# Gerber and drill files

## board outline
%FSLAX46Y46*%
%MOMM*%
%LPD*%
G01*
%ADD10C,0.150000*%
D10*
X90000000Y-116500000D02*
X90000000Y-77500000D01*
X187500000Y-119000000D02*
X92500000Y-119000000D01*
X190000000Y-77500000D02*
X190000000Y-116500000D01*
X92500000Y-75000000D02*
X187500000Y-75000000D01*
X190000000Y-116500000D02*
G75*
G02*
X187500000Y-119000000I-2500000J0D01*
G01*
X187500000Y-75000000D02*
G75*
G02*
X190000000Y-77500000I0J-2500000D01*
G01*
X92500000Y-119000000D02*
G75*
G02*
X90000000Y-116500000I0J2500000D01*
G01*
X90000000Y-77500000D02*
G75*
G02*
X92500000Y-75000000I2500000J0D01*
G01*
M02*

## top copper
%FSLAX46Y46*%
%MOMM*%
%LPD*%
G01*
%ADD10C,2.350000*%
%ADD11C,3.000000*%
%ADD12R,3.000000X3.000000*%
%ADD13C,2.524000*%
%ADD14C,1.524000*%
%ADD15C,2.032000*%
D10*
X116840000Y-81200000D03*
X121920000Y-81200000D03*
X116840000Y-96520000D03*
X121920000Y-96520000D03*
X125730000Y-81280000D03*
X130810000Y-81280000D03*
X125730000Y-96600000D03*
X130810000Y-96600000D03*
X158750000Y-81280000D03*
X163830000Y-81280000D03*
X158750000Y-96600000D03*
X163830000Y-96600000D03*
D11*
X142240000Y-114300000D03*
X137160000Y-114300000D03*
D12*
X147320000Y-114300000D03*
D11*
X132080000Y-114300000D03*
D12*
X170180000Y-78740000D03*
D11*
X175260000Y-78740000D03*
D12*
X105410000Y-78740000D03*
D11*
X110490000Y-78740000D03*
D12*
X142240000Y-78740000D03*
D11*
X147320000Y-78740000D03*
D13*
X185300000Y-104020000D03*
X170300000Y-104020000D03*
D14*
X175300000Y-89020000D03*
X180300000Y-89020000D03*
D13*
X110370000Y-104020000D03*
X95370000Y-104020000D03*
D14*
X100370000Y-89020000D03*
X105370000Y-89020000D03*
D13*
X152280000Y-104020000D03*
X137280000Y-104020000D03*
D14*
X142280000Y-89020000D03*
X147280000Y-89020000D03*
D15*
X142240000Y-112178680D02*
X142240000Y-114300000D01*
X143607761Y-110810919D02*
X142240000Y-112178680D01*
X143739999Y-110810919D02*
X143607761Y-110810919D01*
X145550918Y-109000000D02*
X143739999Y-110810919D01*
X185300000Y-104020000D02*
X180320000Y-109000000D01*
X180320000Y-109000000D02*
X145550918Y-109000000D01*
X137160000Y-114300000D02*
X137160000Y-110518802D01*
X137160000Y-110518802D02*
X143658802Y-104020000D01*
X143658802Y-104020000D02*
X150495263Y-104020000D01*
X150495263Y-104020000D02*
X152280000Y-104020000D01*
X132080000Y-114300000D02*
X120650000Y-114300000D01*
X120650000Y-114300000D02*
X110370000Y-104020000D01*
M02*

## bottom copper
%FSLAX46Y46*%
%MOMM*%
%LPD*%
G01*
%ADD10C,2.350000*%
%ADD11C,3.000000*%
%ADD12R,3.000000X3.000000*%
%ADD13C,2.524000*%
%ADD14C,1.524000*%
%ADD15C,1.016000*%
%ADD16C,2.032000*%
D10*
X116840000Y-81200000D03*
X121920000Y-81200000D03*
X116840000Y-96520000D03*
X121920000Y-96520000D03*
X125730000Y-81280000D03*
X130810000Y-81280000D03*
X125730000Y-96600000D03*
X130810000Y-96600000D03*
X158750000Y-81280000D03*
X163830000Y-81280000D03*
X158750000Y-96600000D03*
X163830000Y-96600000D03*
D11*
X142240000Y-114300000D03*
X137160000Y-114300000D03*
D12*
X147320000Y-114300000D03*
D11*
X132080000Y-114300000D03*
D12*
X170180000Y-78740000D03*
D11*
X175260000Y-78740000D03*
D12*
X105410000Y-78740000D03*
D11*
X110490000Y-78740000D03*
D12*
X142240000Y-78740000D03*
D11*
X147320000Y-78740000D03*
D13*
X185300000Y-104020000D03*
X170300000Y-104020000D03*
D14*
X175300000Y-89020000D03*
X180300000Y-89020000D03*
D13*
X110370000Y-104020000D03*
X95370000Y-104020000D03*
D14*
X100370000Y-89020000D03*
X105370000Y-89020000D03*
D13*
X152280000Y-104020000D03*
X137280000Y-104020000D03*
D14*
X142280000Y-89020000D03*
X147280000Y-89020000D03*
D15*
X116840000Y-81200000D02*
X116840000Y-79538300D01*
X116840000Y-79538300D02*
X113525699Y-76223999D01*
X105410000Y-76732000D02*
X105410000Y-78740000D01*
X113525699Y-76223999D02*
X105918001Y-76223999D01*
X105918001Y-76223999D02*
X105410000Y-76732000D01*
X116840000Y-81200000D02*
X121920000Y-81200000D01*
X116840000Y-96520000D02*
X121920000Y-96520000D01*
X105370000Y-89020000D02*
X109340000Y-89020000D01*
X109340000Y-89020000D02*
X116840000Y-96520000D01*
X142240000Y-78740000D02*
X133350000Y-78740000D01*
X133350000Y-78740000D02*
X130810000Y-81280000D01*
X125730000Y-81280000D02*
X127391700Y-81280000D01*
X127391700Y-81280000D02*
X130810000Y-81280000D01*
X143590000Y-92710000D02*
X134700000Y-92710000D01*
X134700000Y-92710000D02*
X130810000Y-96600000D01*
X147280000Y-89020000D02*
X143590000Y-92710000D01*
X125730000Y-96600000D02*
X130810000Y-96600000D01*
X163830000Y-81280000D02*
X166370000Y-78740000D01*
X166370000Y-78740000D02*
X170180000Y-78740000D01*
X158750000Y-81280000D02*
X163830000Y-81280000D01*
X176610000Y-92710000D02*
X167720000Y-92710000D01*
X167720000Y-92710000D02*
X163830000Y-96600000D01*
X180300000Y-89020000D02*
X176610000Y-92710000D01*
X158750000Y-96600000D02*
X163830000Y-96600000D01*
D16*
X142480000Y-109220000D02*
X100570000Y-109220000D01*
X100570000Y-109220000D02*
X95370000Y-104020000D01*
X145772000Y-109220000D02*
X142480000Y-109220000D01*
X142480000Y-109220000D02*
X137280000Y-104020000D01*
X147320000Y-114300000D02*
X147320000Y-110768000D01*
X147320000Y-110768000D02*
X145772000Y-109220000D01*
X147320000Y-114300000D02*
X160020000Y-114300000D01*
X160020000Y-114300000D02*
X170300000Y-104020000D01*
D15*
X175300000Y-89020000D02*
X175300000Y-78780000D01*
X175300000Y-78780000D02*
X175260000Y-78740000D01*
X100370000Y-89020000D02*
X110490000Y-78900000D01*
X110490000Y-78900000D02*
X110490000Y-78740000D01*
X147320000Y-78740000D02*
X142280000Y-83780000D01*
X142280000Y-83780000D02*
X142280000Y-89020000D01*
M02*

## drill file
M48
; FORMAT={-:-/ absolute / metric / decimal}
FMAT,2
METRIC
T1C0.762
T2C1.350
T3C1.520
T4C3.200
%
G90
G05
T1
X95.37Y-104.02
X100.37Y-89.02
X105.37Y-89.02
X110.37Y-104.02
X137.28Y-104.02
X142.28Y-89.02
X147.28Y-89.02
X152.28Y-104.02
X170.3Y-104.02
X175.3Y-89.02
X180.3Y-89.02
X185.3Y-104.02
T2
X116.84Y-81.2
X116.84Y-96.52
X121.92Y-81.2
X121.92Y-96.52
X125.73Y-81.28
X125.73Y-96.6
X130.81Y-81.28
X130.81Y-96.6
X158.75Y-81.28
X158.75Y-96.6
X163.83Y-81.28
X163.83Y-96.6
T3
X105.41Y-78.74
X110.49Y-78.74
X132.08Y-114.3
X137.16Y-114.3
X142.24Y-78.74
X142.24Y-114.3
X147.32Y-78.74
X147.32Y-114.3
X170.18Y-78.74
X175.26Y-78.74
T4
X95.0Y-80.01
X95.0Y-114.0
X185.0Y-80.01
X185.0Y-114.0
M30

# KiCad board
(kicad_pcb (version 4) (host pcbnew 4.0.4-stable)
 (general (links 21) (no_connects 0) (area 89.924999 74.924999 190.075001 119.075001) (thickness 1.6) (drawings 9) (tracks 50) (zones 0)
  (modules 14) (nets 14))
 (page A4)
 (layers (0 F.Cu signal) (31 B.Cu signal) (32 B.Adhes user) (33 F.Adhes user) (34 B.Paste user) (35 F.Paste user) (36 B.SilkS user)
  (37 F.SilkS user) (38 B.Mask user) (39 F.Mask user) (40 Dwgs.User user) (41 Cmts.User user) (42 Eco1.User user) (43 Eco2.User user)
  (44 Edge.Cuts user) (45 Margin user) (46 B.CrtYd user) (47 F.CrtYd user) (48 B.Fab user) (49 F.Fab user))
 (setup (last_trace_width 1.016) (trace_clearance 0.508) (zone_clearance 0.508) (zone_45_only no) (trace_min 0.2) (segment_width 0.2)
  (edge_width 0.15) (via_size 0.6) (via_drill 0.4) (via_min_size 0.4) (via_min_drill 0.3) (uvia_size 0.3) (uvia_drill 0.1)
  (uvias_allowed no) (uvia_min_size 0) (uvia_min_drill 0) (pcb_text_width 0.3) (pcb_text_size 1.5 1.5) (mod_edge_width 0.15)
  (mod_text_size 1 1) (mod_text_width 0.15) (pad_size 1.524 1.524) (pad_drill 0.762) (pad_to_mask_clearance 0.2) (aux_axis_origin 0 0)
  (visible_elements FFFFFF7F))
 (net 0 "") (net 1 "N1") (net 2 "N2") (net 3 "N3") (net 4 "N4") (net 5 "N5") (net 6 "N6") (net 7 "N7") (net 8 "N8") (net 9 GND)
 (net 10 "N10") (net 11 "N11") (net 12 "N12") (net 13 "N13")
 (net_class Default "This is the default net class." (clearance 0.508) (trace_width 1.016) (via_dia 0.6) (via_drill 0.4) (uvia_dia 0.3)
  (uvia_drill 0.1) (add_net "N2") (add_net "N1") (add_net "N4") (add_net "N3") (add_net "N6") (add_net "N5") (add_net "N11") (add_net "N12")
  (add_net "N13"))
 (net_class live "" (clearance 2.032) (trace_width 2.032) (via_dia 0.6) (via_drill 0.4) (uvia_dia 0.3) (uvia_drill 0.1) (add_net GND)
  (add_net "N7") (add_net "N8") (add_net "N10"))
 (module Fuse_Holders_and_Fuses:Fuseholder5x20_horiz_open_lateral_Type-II (layer F.Cu) (at 116.84 96.52 90)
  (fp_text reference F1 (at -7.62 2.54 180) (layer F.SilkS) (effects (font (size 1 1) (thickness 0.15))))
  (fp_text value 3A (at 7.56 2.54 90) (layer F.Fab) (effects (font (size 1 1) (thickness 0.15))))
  (pad 2 thru_hole circle (at 15.32 0 90) (size 2.35 2.35) (drill 1.35) (layers *.Cu *.Mask) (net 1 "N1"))
  (pad 2 thru_hole circle (at 15.32 5.08 90) (size 2.35 2.35) (drill 1.35) (layers *.Cu *.Mask) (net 1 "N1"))
  (pad 1 thru_hole circle (at 0 0 90) (size 2.35 2.35) (drill 1.35) (layers *.Cu *.Mask) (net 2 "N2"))
  (pad 1 thru_hole circle (at 0 5.08 90) (size 2.35 2.35) (drill 1.35) (layers *.Cu *.Mask) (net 2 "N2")))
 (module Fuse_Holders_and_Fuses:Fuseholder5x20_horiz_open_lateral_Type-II (layer F.Cu) (at 125.73 96.6 90)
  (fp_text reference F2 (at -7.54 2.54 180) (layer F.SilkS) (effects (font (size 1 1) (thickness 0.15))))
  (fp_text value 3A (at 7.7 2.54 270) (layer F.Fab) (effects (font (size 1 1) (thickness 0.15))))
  (pad 2 thru_hole circle (at 15.32 0 90) (size 2.35 2.35) (drill 1.35) (layers *.Cu *.Mask) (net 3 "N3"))
  (pad 2 thru_hole circle (at 15.32 5.08 90) (size 2.35 2.35) (drill 1.35) (layers *.Cu *.Mask) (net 3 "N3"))
  (pad 1 thru_hole circle (at 0 0 90) (size 2.35 2.35) (drill 1.35) (layers *.Cu *.Mask) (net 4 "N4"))
  (pad 1 thru_hole circle (at 0 5.08 90) (size 2.35 2.35) (drill 1.35) (layers *.Cu *.Mask) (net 4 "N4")))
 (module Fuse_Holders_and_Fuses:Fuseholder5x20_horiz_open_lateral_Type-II (layer F.Cu) (at 158.75 96.6 90)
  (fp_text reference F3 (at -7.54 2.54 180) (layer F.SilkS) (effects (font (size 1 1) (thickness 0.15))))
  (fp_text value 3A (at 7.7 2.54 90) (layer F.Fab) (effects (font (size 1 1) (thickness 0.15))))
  (pad 2 thru_hole circle (at 15.32 0 90) (size 2.35 2.35) (drill 1.35) (layers *.Cu *.Mask) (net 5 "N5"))
  (pad 2 thru_hole circle (at 15.32 5.08 90) (size 2.35 2.35) (drill 1.35) (layers *.Cu *.Mask) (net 5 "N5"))
  (pad 1 thru_hole circle (at 0 0 90) (size 2.35 2.35) (drill 1.35) (layers *.Cu *.Mask) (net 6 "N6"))
  (pad 1 thru_hole circle (at 0 5.08 90) (size 2.35 2.35) (drill 1.35) (layers *.Cu *.Mask) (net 6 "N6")))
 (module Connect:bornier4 (layer F.Cu) (at 147.32 114.3 180)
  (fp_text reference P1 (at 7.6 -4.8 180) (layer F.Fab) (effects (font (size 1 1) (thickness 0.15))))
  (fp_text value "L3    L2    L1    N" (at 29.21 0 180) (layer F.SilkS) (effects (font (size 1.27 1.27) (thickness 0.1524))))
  (pad 2 thru_hole circle (at 5.08 0 180) (size 3 3) (drill 1.52) (layers *.Cu *.Mask) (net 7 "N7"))
  (pad 3 thru_hole circle (at 10.16 0 180) (size 3 3) (drill 1.52) (layers *.Cu *.Mask) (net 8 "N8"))
  (pad 1 thru_hole rect (at 0 0 180) (size 3 3) (drill 1.52) (layers *.Cu *.Mask) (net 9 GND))
  (pad 4 thru_hole circle (at 15.24 0 180) (size 3 3) (drill 1.52) (layers *.Cu *.Mask) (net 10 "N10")))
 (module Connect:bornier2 (layer F.Cu) (at 170.18 78.74)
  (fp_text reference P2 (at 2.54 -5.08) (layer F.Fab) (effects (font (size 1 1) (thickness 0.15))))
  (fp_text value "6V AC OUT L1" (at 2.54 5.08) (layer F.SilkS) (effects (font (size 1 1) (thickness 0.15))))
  (pad 1 thru_hole rect (at 0 0) (size 3 3) (drill 1.52) (layers *.Cu *.Mask) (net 5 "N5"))
  (pad 2 thru_hole circle (at 5.08 0) (size 3 3) (drill 1.52) (layers *.Cu *.Mask) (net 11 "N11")))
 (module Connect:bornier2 (layer F.Cu) (at 105.41 78.74)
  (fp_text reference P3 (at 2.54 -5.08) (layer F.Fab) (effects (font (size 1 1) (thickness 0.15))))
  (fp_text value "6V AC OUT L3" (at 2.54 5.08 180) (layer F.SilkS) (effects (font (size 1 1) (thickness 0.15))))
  (pad 1 thru_hole rect (at 0 0) (size 3 3) (drill 1.52) (layers *.Cu *.Mask) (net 1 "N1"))
  (pad 2 thru_hole circle (at 5.08 0) (size 3 3) (drill 1.52) (layers *.Cu *.Mask) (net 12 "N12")))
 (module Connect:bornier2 (layer F.Cu) (at 142.24 78.74)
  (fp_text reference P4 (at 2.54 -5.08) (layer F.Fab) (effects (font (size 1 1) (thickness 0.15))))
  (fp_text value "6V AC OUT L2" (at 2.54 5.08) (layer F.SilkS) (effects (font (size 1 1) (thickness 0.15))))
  (pad 1 thru_hole rect (at 0 0) (size 3 3) (drill 1.52) (layers *.Cu *.Mask) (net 3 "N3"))
  (pad 2 thru_hole circle (at 5.08 0) (size 3 3) (drill 1.52) (layers *.Cu *.Mask) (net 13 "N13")))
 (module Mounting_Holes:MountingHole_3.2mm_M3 (layer F.Cu) (at 185 80.01 90)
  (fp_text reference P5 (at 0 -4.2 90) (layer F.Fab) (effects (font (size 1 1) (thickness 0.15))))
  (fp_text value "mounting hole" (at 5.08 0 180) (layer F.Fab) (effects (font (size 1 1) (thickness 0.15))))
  (pad 1 np_thru_hole circle (at 0 0 90) (size 3.2 3.2) (drill 3.2) (layers *.Cu *.Mask)))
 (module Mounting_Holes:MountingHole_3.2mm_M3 (layer F.Cu) (at 185 114 90)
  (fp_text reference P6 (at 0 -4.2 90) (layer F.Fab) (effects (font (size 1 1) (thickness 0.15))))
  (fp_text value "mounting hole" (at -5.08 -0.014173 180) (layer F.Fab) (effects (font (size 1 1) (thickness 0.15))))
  (pad 1 np_thru_hole circle (at 0 0 90) (size 3.2 3.2) (drill 3.2) (layers *.Cu *.Mask)))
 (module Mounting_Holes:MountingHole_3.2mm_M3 (layer F.Cu) (at 95 114 90)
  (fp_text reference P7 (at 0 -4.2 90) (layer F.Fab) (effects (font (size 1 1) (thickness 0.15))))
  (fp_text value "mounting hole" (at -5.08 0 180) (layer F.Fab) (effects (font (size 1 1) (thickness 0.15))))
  (pad 1 np_thru_hole circle (at 0 0 90) (size 3.2 3.2) (drill 3.2) (layers *.Cu *.Mask)))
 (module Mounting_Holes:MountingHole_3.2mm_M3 (layer F.Cu) (at 95 80.01 90)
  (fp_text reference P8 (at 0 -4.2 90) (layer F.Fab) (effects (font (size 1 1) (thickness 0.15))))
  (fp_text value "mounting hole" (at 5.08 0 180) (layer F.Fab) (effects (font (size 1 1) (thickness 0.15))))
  (pad 1 np_thru_hole circle (at 0 0 90) (size 3.2 3.2) (drill 3.2) (layers *.Cu *.Mask)))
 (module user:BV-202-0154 (layer F.Cu) (at 177.8 96.52 90)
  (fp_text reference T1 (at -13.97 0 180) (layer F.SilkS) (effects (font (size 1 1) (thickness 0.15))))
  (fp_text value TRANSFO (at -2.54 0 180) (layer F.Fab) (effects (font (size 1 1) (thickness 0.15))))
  (pad 1 thru_hole circle (at -7.5 7.5 90) (size 2.524 2.524) (drill 0.762) (layers *.Cu *.Mask) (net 7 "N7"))
  (pad 2 thru_hole circle (at -7.5 -7.5 90) (size 2.524 2.524) (drill 0.762) (layers *.Cu *.Mask) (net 9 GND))
  (pad 3 thru_hole circle (at 7.5 -2.5 90) (size 1.524 1.524) (drill 0.762) (layers *.Cu *.Mask) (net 11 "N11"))
  (pad 4 thru_hole circle (at 7.5 2.5 90) (size 1.524 1.524) (drill 0.762) (layers *.Cu *.Mask) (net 6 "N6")))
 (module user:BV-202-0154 (layer F.Cu) (at 102.87 96.52 90)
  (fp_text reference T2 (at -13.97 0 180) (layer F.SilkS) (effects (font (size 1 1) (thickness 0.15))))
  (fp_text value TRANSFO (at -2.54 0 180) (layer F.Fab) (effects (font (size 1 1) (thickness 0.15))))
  (pad 1 thru_hole circle (at -7.5 7.5 90) (size 2.524 2.524) (drill 0.762) (layers *.Cu *.Mask) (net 10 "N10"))
  (pad 2 thru_hole circle (at -7.5 -7.5 90) (size 2.524 2.524) (drill 0.762) (layers *.Cu *.Mask) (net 9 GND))
  (pad 3 thru_hole circle (at 7.5 -2.5 90) (size 1.524 1.524) (drill 0.762) (layers *.Cu *.Mask) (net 12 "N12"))
  (pad 4 thru_hole circle (at 7.5 2.5 90) (size 1.524 1.524) (drill 0.762) (layers *.Cu *.Mask) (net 2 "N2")))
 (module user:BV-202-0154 (layer F.Cu) (at 144.78 96.52 90)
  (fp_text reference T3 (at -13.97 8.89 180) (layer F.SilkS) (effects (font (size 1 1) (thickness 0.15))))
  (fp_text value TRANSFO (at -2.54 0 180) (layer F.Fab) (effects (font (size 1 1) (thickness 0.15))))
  (pad 1 thru_hole circle (at -7.5 7.5 90) (size 2.524 2.524) (drill 0.762) (layers *.Cu *.Mask) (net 8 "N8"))
  (pad 2 thru_hole circle (at -7.5 -7.5 90) (size 2.524 2.524) (drill 0.762) (layers *.Cu *.Mask) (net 9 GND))
  (pad 3 thru_hole circle (at 7.5 -2.5 90) (size 1.524 1.524) (drill 0.762) (layers *.Cu *.Mask) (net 13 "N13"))
  (pad 4 thru_hole circle (at 7.5 2.5 90) (size 1.524 1.524) (drill 0.762) (layers *.Cu *.Mask) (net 4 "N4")))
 (gr_line (start 90 116.5) (end 90 77.5) (layer Edge.Cuts) (width 0.15))
 (gr_line (start 187.5 119) (end 92.5 119) (layer Edge.Cuts) (width 0.15))
 (gr_line (start 190 77.5) (end 190 116.5) (layer Edge.Cuts) (width 0.15))
 (gr_line (start 92.5 75) (end 187.5 75) (layer Edge.Cuts) (width 0.15))
 (gr_arc (start 187.5 116.5) (end 190 116.5) (angle 90) (layer Edge.Cuts) (width 0.15))
 (gr_arc (start 187.5 77.5) (end 187.5 75) (angle 90) (layer Edge.Cuts) (width 0.15))
 (gr_arc (start 92.5 116.5) (end 92.5 119) (angle 90) (layer Edge.Cuts) (width 0.15))
 (gr_arc (start 92.5 77.5) (end 90 77.5) (angle 90) (layer Edge.Cuts) (width 0.15))
 (segment (start 116.84 81.2) (end 116.84 79.5383) (width 1.016) (layer B.Cu) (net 1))
 (segment (start 116.84 79.5383) (end 113.525699 76.223999) (width 1.016) (layer B.Cu) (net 1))
 (segment (start 105.41 76.732) (end 105.41 78.74) (width 1.016) (layer B.Cu) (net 1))
 (segment (start 113.525699 76.223999) (end 105.918001 76.223999) (width 1.016) (layer B.Cu) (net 1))
 (segment (start 105.918001 76.223999) (end 105.41 76.732) (width 1.016) (layer B.Cu) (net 1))
 (segment (start 116.84 81.2) (end 121.92 81.2) (width 1.016) (layer B.Cu) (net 1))
 (segment (start 116.84 96.52) (end 121.92 96.52) (width 1.016) (layer B.Cu) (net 2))
 (segment (start 105.37 89.02) (end 109.34 89.02) (width 1.016) (layer B.Cu) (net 2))
 (segment (start 109.34 89.02) (end 116.84 96.52) (width 1.016) (layer B.Cu) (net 2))
 (segment (start 142.24 78.74) (end 133.35 78.74) (width 1.016) (layer B.Cu) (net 3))
 (segment (start 133.35 78.74) (end 130.81 81.28) (width 1.016) (layer B.Cu) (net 3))
 (segment (start 125.73 81.28) (end 127.3917 81.28) (width 1.016) (layer B.Cu) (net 3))
 (segment (start 127.3917 81.28) (end 130.81 81.28) (width 1.016) (layer B.Cu) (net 3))
 (segment (start 143.59 92.71) (end 134.7 92.71) (width 1.016) (layer B.Cu) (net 4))
 (segment (start 134.7 92.71) (end 130.81 96.6) (width 1.016) (layer B.Cu) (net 4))
 (segment (start 147.28 89.02) (end 143.59 92.71) (width 1.016) (layer B.Cu) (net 4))
 (segment (start 125.73 96.6) (end 130.81 96.6) (width 1.016) (layer B.Cu) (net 4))
 (segment (start 163.83 81.28) (end 166.37 78.74) (width 1.016) (layer B.Cu) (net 5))
 (segment (start 166.37 78.74) (end 170.18 78.74) (width 1.016) (layer B.Cu) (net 5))
 (segment (start 158.75 81.28) (end 163.83 81.28) (width 1.016) (layer B.Cu) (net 5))
 (segment (start 176.61 92.71) (end 167.72 92.71) (width 1.016) (layer B.Cu) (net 6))
 (segment (start 167.72 92.71) (end 163.83 96.6) (width 1.016) (layer B.Cu) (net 6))
 (segment (start 180.3 89.02) (end 176.61 92.71) (width 1.016) (layer B.Cu) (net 6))
 (segment (start 158.75 96.6) (end 163.83 96.6) (width 1.016) (layer B.Cu) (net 6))
 (segment (start 142.24 112.17868) (end 142.24 114.3) (width 2.032) (layer F.Cu) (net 7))
 (segment (start 143.607761 110.810919) (end 142.24 112.17868) (width 2.032) (layer F.Cu) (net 7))
 (segment (start 143.739999 110.810919) (end 143.607761 110.810919) (width 2.032) (layer F.Cu) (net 7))
 (segment (start 145.550918 109) (end 143.739999 110.810919) (width 2.032) (layer F.Cu) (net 7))
 (segment (start 185.3 104.02) (end 180.32 109) (width 2.032) (layer F.Cu) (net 7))
 (segment (start 180.32 109) (end 145.550918 109) (width 2.032) (layer F.Cu) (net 7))
 (segment (start 137.16 114.3) (end 137.16 110.518802) (width 2.032) (layer F.Cu) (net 8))
 (segment (start 137.16 110.518802) (end 143.658802 104.02) (width 2.032) (layer F.Cu) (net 8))
 (segment (start 143.658802 104.02) (end 150.495263 104.02) (width 2.032) (layer F.Cu) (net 8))
 (segment (start 150.495263 104.02) (end 152.28 104.02) (width 2.032) (layer F.Cu) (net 8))
 (segment (start 142.48 109.22) (end 100.57 109.22) (width 2.032) (layer B.Cu) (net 9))
 (segment (start 100.57 109.22) (end 95.37 104.02) (width 2.032) (layer B.Cu) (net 9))
 (segment (start 145.772 109.22) (end 142.48 109.22) (width 2.032) (layer B.Cu) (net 9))
 (segment (start 142.48 109.22) (end 137.28 104.02) (width 2.032) (layer B.Cu) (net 9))
 (segment (start 147.32 114.3) (end 147.32 110.768) (width 2.032) (layer B.Cu) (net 9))
 (segment (start 147.32 110.768) (end 145.772 109.22) (width 2.032) (layer B.Cu) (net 9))
 (segment (start 147.32 114.3) (end 160.02 114.3) (width 2.032) (layer B.Cu) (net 9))
 (segment (start 160.02 114.3) (end 170.3 104.02) (width 2.032) (layer B.Cu) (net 9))
 (segment (start 132.08 114.3) (end 120.65 114.3) (width 2.032) (layer F.Cu) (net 10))
 (segment (start 120.65 114.3) (end 110.37 104.02) (width 2.032) (layer F.Cu) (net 10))
 (segment (start 175.3 89.02) (end 175.3 78.78) (width 1.016) (layer B.Cu) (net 11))
 (segment (start 175.3 78.78) (end 175.26 78.74) (width 1.016) (layer B.Cu) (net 11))
 (segment (start 100.37 89.02) (end 110.49 78.9) (width 1.016) (layer B.Cu) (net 12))
 (segment (start 110.49 78.9) (end 110.49 78.74) (width 1.016) (layer B.Cu) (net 12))
 (segment (start 147.32 78.74) (end 142.28 83.78) (width 1.016) (layer B.Cu) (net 13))
 (segment (start 142.28 83.78) (end 142.28 89.02) (width 1.016) (layer B.Cu) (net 13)))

